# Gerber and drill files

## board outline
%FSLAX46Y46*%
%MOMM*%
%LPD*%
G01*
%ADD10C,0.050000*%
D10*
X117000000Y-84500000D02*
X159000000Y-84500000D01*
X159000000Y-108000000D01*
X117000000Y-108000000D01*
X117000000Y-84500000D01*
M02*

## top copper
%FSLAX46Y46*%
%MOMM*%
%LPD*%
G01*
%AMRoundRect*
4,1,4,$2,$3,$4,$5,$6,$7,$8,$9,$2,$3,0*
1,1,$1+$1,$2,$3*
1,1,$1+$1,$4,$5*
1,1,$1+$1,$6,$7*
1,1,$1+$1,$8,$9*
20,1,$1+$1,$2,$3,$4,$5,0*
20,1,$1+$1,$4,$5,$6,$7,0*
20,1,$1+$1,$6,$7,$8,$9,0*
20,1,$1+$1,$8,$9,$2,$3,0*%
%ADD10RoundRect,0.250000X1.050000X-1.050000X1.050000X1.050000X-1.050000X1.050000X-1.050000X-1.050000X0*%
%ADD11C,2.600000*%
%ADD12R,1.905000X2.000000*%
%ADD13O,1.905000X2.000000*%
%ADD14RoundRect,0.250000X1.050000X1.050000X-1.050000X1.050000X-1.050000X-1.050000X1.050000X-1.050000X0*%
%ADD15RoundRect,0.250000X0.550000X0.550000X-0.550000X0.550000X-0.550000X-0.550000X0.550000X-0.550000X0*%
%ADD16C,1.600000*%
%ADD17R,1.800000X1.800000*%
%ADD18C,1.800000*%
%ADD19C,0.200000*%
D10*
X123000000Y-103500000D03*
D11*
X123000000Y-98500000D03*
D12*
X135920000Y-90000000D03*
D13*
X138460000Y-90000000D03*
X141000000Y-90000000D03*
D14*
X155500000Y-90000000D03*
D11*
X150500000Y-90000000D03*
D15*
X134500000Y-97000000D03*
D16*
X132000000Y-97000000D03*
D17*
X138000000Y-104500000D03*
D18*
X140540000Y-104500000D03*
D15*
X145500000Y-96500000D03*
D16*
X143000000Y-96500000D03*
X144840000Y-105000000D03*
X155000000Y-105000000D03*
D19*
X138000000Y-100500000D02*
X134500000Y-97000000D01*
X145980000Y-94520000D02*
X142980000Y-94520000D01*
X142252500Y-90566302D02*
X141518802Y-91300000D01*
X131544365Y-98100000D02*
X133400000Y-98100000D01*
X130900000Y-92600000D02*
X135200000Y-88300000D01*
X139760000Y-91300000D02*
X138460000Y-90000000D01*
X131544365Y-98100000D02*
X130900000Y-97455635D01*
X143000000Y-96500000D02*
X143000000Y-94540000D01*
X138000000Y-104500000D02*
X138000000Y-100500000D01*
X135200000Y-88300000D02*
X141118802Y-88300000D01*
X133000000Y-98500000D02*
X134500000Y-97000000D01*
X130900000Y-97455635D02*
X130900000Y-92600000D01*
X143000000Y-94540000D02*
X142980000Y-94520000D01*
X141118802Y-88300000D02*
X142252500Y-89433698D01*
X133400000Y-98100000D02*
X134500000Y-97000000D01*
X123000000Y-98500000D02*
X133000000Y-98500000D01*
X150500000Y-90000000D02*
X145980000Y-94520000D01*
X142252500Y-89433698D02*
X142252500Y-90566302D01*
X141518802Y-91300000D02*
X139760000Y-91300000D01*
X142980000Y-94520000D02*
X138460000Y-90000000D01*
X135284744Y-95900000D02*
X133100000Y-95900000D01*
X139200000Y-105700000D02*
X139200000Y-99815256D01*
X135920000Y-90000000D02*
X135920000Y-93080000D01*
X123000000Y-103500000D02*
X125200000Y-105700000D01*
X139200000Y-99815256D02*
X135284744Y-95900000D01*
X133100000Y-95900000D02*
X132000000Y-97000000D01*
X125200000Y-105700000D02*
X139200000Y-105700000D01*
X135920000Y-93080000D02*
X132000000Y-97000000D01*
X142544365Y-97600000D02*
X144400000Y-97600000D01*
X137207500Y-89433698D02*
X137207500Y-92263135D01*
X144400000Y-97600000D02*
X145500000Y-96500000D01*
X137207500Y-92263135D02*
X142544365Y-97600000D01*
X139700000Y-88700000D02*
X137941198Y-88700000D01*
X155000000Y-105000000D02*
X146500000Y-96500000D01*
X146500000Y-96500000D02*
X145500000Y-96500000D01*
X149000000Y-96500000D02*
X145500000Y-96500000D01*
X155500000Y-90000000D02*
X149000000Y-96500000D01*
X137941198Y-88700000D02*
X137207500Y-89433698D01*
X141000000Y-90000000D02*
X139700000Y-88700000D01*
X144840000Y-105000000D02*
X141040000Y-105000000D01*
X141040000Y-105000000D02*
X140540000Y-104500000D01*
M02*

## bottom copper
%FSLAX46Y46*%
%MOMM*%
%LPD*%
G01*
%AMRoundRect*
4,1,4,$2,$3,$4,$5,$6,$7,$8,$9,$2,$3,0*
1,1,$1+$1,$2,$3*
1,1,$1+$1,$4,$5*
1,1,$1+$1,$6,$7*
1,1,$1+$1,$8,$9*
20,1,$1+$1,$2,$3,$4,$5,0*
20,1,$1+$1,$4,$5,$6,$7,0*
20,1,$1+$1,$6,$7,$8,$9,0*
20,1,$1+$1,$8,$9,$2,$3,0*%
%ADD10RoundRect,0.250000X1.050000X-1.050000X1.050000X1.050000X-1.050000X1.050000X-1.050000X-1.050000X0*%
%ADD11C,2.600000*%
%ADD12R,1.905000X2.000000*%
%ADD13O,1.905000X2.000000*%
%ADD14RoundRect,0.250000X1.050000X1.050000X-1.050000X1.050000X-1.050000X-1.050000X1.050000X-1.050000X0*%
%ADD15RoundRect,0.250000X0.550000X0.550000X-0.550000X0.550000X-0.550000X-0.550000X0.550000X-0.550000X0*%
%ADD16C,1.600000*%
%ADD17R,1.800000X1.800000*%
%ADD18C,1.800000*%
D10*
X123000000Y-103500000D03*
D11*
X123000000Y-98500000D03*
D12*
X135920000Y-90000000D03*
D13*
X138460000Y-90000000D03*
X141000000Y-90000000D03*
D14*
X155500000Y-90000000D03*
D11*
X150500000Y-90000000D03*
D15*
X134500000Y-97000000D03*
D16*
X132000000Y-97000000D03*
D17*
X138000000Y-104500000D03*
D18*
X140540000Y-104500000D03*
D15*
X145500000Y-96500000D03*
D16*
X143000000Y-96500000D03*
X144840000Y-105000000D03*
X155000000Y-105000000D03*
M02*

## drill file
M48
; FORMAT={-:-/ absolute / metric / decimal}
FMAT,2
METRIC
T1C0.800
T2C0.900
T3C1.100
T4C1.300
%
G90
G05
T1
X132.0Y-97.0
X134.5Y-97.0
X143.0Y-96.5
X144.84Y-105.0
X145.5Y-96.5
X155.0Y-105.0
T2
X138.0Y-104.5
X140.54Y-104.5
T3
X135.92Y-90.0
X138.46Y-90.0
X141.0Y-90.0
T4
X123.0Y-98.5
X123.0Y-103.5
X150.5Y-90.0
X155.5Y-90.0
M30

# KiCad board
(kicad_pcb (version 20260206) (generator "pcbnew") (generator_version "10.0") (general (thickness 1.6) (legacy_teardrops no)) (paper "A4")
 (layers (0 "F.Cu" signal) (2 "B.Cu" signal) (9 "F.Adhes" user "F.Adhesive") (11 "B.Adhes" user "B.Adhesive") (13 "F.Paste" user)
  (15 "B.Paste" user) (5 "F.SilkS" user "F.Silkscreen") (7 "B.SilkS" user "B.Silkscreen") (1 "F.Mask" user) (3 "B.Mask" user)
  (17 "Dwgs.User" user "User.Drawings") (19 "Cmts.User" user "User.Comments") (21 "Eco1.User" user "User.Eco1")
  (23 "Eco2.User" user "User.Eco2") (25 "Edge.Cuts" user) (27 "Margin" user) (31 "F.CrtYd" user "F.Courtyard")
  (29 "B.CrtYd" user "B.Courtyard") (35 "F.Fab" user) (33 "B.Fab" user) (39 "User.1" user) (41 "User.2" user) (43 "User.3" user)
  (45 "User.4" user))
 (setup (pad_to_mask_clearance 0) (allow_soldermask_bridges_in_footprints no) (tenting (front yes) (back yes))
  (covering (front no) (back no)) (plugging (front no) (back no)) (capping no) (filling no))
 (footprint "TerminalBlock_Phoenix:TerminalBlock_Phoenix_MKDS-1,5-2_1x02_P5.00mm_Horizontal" (layer "F.Cu") (at 123 103.5 90)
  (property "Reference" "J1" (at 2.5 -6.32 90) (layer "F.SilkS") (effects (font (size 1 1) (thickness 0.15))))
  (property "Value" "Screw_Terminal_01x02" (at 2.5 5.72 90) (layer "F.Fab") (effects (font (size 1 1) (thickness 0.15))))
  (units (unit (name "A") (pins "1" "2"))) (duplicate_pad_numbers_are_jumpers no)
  (pad "1" thru_hole roundrect (at 0 0 90) (size 2.6 2.6) (drill 1.3) (layers "*.Cu" "*.Mask") (remove_unused_layers no)
   (roundrect_rratio 0.096154) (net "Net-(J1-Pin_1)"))
  (pad "2" thru_hole circle (at 5 0 90) (size 2.6 2.6) (drill 1.3) (layers "*.Cu" "*.Mask") (remove_unused_layers no) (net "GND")))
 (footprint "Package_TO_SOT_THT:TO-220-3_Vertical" (layer "F.Cu") (at 135.92 90)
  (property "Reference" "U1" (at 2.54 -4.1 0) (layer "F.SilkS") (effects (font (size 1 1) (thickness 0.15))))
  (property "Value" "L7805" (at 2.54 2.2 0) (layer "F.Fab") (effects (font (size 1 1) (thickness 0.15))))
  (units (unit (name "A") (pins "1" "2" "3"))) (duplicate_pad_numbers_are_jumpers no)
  (pad "1" thru_hole rect (at 0 0) (size 1.905 2) (drill 1.1) (layers "*.Cu" "*.Mask") (remove_unused_layers no) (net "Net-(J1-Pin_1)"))
  (pad "2" thru_hole oval (at 2.54 0) (size 1.905 2) (drill 1.1) (layers "*.Cu" "*.Mask") (remove_unused_layers no) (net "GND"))
  (pad "3" thru_hole oval (at 5.08 0) (size 1.905 2) (drill 1.1) (layers "*.Cu" "*.Mask") (remove_unused_layers no) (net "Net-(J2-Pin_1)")))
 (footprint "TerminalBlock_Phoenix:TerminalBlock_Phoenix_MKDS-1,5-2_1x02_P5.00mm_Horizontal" (layer "F.Cu") (at 155.5 90 180)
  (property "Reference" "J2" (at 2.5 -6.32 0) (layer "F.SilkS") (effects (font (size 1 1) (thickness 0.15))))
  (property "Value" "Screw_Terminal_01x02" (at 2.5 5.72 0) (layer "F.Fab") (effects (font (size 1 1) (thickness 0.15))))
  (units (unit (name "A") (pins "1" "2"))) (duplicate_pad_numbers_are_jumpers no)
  (pad "1" thru_hole roundrect (at 0 0 180) (size 2.6 2.6) (drill 1.3) (layers "*.Cu" "*.Mask") (remove_unused_layers no)
   (roundrect_rratio 0.096154) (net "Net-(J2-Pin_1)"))
  (pad "2" thru_hole circle (at 5 0 180) (size 2.6 2.6) (drill 1.3) (layers "*.Cu" "*.Mask") (remove_unused_layers no) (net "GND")))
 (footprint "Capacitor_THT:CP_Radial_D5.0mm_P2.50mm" (layer "F.Cu") (at 134.5 97 180)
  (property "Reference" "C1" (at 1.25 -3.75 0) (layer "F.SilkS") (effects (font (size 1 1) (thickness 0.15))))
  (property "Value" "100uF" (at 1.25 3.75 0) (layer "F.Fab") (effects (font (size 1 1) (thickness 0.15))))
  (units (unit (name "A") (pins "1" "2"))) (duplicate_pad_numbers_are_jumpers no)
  (pad "1" thru_hole roundrect (at 0 0 180) (size 1.6 1.6) (drill 0.8) (layers "*.Cu" "*.Mask") (remove_unused_layers no)
   (roundrect_rratio 0.15625) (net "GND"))
  (pad "2" thru_hole circle (at 2.5 0 180) (size 1.6 1.6) (drill 0.8) (layers "*.Cu" "*.Mask") (remove_unused_layers no)
   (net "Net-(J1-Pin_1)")))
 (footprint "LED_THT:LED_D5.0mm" (layer "F.Cu") (at 138 104.5)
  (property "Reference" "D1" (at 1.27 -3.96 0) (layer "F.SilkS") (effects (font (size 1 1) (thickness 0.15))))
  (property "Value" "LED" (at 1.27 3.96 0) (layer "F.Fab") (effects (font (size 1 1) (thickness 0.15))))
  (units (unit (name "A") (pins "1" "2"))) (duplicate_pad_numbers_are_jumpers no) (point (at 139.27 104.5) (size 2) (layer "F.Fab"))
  (pad "1" thru_hole rect (at 0 0) (size 1.8 1.8) (drill 0.9) (layers "*.Cu" "*.Mask") (remove_unused_layers no) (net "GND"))
  (pad "2" thru_hole circle (at 2.54 0) (size 1.8 1.8) (drill 0.9) (layers "*.Cu" "*.Mask") (remove_unused_layers no) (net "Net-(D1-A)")))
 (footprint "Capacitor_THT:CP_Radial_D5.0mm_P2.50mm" (layer "F.Cu") (at 145.5 96.5 180)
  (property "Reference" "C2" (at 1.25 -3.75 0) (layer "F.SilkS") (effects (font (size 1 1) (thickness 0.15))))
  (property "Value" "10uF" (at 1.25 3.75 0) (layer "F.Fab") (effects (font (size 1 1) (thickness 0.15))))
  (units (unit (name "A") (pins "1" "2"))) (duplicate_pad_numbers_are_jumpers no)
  (pad "1" thru_hole roundrect (at 0 0 180) (size 1.6 1.6) (drill 0.8) (layers "*.Cu" "*.Mask") (remove_unused_layers no)
   (roundrect_rratio 0.15625) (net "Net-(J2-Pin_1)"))
  (pad "2" thru_hole circle (at 2.5 0 180) (size 1.6 1.6) (drill 0.8) (layers "*.Cu" "*.Mask") (remove_unused_layers no) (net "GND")))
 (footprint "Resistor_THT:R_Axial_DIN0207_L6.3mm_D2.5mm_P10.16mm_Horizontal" (layer "F.Cu") (at 144.84 105)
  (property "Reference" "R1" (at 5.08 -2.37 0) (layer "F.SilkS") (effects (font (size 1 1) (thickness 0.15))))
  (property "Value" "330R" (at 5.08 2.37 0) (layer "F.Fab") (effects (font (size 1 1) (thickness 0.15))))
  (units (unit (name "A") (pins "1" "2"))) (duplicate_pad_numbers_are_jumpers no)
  (pad "1" thru_hole circle (at 0 0) (size 1.6 1.6) (drill 0.8) (layers "*.Cu" "*.Mask") (remove_unused_layers no) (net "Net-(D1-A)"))
  (pad "2" thru_hole circle (at 10.16 0) (size 1.6 1.6) (drill 0.8) (layers "*.Cu" "*.Mask") (remove_unused_layers no)
   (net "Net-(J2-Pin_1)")))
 (gr_rect (start 117 84.5) (end 159 108) (stroke (width 0.05) (type default)) (fill no) (layer "Edge.Cuts"))
 (segment (start 138 100.5) (end 134.5 97) (width 0.2) (layer "F.Cu") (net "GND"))
 (segment (start 145.98 94.52) (end 142.98 94.52) (width 0.2) (layer "F.Cu") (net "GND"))
 (segment (start 142.2525 90.566302) (end 141.518802 91.3) (width 0.2) (layer "F.Cu") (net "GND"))
 (segment (start 131.544365 98.1) (end 133.4 98.1) (width 0.2) (layer "F.Cu") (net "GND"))
 (segment (start 130.9 92.6) (end 135.2 88.3) (width 0.2) (layer "F.Cu") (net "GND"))
 (segment (start 139.76 91.3) (end 138.46 90) (width 0.2) (layer "F.Cu") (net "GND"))
 (segment (start 131.544365 98.1) (end 130.9 97.455635) (width 0.2) (layer "F.Cu") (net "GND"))
 (segment (start 143 96.5) (end 143 94.54) (width 0.2) (layer "F.Cu") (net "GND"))
 (segment (start 138 104.5) (end 138 100.5) (width 0.2) (layer "F.Cu") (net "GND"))
 (segment (start 135.2 88.3) (end 141.118802 88.3) (width 0.2) (layer "F.Cu") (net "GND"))
 (segment (start 133 98.5) (end 134.5 97) (width 0.2) (layer "F.Cu") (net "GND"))
 (segment (start 130.9 97.455635) (end 130.9 92.6) (width 0.2) (layer "F.Cu") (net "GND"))
 (segment (start 143 94.54) (end 142.98 94.52) (width 0.2) (layer "F.Cu") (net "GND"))
 (segment (start 141.118802 88.3) (end 142.2525 89.433698) (width 0.2) (layer "F.Cu") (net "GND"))
 (segment (start 133.4 98.1) (end 134.5 97) (width 0.2) (layer "F.Cu") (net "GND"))
 (segment (start 123 98.5) (end 133 98.5) (width 0.2) (layer "F.Cu") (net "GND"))
 (segment (start 150.5 90) (end 145.98 94.52) (width 0.2) (layer "F.Cu") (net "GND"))
 (segment (start 142.2525 89.433698) (end 142.2525 90.566302) (width 0.2) (layer "F.Cu") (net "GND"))
 (segment (start 141.518802 91.3) (end 139.76 91.3) (width 0.2) (layer "F.Cu") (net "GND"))
 (segment (start 142.98 94.52) (end 138.46 90) (width 0.2) (layer "F.Cu") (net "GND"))
 (segment (start 135.284744 95.9) (end 133.1 95.9) (width 0.2) (layer "F.Cu") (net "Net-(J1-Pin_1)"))
 (segment (start 139.2 105.7) (end 139.2 99.815256) (width 0.2) (layer "F.Cu") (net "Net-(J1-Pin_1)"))
 (segment (start 135.92 90) (end 135.92 93.08) (width 0.2) (layer "F.Cu") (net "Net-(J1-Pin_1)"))
 (segment (start 123 103.5) (end 125.2 105.7) (width 0.2) (layer "F.Cu") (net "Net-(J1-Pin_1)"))
 (segment (start 139.2 99.815256) (end 135.284744 95.9) (width 0.2) (layer "F.Cu") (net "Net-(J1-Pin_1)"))
 (segment (start 133.1 95.9) (end 132 97) (width 0.2) (layer "F.Cu") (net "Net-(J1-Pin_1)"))
 (segment (start 125.2 105.7) (end 139.2 105.7) (width 0.2) (layer "F.Cu") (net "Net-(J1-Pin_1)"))
 (segment (start 135.92 93.08) (end 132 97) (width 0.2) (layer "F.Cu") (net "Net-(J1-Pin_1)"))
 (segment (start 142.544365 97.6) (end 144.4 97.6) (width 0.2) (layer "F.Cu") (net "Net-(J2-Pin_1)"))
 (segment (start 137.2075 89.433698) (end 137.2075 92.263135) (width 0.2) (layer "F.Cu") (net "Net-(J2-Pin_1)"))
 (segment (start 144.4 97.6) (end 145.5 96.5) (width 0.2) (layer "F.Cu") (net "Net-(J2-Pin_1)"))
 (segment (start 137.2075 92.263135) (end 142.544365 97.6) (width 0.2) (layer "F.Cu") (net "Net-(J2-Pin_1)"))
 (segment (start 139.7 88.7) (end 137.941198 88.7) (width 0.2) (layer "F.Cu") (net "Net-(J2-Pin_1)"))
 (segment (start 155 105) (end 146.5 96.5) (width 0.2) (layer "F.Cu") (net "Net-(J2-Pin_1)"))
 (segment (start 146.5 96.5) (end 145.5 96.5) (width 0.2) (layer "F.Cu") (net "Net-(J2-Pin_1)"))
 (segment (start 149 96.5) (end 145.5 96.5) (width 0.2) (layer "F.Cu") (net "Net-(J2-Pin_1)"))
 (segment (start 155.5 90) (end 149 96.5) (width 0.2) (layer "F.Cu") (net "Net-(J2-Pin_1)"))
 (segment (start 137.941198 88.7) (end 137.2075 89.433698) (width 0.2) (layer "F.Cu") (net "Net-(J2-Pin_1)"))
 (segment (start 141 90) (end 139.7 88.7) (width 0.2) (layer "F.Cu") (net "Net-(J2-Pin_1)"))
 (segment (start 144.84 105) (end 141.04 105) (width 0.2) (layer "F.Cu") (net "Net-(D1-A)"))
 (segment (start 141.04 105) (end 140.54 104.5) (width 0.2) (layer "F.Cu") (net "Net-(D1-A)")))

